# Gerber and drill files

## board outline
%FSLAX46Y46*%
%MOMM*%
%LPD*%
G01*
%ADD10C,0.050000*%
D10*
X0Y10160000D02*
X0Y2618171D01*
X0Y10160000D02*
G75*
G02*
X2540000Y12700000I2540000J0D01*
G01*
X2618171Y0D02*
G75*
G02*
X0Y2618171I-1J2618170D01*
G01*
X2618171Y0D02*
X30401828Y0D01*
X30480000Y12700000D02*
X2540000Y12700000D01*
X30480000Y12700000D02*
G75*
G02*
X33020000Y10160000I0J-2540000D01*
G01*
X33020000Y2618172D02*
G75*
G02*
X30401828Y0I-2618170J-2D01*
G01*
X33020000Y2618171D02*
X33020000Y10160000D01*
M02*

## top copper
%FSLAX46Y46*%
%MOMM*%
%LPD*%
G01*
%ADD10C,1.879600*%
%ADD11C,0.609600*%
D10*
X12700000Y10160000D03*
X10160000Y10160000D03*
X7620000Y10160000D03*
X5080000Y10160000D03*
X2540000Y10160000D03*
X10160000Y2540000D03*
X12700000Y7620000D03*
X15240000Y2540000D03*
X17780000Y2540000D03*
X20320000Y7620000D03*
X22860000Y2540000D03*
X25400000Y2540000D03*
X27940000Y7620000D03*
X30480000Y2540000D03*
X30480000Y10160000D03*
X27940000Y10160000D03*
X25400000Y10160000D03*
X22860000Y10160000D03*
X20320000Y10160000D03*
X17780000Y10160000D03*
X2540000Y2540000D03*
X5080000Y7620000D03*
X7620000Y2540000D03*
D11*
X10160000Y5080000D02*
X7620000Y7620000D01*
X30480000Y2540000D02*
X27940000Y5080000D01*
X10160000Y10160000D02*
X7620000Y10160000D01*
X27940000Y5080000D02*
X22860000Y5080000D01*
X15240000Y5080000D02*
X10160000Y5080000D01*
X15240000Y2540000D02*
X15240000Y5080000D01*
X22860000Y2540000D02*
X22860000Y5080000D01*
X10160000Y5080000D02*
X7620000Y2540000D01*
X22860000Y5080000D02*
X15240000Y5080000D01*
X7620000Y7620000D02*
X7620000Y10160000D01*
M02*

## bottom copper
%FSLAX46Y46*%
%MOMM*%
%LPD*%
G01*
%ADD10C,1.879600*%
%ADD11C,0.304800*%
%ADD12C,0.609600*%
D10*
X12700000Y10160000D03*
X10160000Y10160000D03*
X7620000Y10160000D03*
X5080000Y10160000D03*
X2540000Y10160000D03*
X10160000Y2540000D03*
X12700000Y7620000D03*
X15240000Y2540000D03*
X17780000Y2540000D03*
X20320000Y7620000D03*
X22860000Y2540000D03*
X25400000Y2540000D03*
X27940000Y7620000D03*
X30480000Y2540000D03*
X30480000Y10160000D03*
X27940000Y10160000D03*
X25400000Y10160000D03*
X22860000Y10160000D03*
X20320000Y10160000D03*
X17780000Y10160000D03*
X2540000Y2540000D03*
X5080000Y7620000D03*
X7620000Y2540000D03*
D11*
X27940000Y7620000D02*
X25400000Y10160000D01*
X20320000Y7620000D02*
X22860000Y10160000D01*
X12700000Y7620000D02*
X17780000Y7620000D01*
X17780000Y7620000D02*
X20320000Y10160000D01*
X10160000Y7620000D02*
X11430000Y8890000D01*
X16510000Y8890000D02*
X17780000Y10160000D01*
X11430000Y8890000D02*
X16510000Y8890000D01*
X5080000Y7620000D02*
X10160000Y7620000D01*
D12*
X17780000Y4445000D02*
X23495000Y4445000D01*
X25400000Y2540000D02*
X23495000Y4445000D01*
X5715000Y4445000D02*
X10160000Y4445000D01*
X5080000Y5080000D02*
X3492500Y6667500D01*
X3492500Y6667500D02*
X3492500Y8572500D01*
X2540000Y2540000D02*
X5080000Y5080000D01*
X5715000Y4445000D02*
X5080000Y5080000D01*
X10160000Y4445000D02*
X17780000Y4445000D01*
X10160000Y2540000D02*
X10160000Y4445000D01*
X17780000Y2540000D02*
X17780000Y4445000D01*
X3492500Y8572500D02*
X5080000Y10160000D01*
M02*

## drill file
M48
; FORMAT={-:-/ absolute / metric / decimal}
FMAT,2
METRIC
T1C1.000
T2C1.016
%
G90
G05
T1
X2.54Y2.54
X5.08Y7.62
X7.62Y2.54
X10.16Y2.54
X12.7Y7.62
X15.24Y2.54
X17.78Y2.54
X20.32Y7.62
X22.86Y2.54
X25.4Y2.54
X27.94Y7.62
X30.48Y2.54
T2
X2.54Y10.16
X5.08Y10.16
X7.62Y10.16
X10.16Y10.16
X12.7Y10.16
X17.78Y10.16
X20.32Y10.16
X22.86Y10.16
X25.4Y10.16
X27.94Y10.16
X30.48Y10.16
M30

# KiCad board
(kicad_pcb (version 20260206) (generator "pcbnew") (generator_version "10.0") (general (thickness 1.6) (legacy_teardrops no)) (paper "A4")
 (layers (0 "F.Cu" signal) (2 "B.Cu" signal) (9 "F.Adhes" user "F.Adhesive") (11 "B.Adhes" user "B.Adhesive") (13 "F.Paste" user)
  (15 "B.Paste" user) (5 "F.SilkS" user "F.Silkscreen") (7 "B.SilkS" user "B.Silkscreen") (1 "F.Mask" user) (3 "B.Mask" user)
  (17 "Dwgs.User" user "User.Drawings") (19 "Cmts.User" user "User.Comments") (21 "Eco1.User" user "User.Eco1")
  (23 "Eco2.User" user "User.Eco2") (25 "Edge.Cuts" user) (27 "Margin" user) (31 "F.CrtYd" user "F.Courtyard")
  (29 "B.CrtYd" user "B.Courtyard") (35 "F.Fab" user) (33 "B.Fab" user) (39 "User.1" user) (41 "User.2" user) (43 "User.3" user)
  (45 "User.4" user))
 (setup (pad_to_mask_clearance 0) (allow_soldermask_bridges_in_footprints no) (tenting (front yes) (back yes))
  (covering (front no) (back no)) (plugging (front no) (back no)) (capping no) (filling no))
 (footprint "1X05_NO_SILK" (layer "F.Cu") (at 12.7 -10.16 180)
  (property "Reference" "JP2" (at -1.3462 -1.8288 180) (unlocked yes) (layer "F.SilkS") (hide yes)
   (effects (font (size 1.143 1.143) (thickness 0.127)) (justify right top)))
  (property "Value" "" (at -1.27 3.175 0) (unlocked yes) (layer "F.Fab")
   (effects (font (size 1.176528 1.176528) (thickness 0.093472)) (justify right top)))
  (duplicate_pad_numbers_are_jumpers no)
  (pad "1" thru_hole circle (at 0 0 270) (size 1.8796 1.8796) (drill 1.016) (layers "*.Cu" "*.Mask") (remove_unused_layers no) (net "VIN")
   (solder_mask_margin 0.0762) (thermal_bridge_angle 0))
  (pad "2" thru_hole circle (at 2.54 0 270) (size 1.8796 1.8796) (drill 1.016) (layers "*.Cu" "*.Mask") (remove_unused_layers no)
   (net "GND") (solder_mask_margin 0.0762) (thermal_bridge_angle 0))
  (pad "3" thru_hole circle (at 5.08 0 270) (size 1.8796 1.8796) (drill 1.016) (layers "*.Cu" "*.Mask") (remove_unused_layers no)
   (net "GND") (solder_mask_margin 0.0762) (thermal_bridge_angle 0))
  (pad "4" thru_hole circle (at 7.62 0 270) (size 1.8796 1.8796) (drill 1.016) (layers "*.Cu" "*.Mask") (remove_unused_layers no) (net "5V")
   (solder_mask_margin 0.0762) (thermal_bridge_angle 0))
  (pad "5" thru_hole circle (at 10.16 0 270) (size 1.8796 1.8796) (drill 1.016) (layers "*.Cu" "*.Mask") (remove_unused_layers no)
   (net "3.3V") (solder_mask_margin 0.0762) (thermal_bridge_angle 0)))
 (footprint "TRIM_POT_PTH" (layer "F.Cu") (at 12.7 -5.08)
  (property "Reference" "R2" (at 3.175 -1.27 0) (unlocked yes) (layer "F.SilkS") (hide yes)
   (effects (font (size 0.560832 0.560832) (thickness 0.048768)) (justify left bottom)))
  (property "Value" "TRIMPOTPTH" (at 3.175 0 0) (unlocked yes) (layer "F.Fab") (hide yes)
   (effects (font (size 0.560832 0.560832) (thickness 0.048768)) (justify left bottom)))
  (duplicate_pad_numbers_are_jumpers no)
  (pad "1" thru_hole circle (at -2.54 2.54 180) (size 1.8796 1.8796) (drill 1) (layers "*.Cu" "*.Mask") (remove_unused_layers no) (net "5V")
   (solder_mask_margin 0.0762) (thermal_bridge_angle 0))
  (pad "2" thru_hole circle (at 0 -2.54 180) (size 1.8796 1.8796) (drill 1) (layers "*.Cu" "*.Mask") (remove_unused_layers no) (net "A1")
   (solder_mask_margin 0.0762) (thermal_bridge_angle 0))
  (pad "3" thru_hole circle (at 2.54 2.54 180) (size 1.8796 1.8796) (drill 1) (layers "*.Cu" "*.Mask") (remove_unused_layers no) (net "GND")
   (solder_mask_margin 0.0762) (thermal_bridge_angle 0)))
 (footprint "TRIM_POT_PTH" (layer "F.Cu") (at 20.32 -5.08)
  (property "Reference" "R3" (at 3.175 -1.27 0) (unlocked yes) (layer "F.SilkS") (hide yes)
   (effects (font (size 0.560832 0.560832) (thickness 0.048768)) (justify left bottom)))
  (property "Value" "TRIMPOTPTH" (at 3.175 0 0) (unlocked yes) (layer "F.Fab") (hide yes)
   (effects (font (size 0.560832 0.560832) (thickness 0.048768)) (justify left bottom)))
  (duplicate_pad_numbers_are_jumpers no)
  (pad "1" thru_hole circle (at -2.54 2.54 180) (size 1.8796 1.8796) (drill 1) (layers "*.Cu" "*.Mask") (remove_unused_layers no) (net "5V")
   (solder_mask_margin 0.0762) (thermal_bridge_angle 0))
  (pad "2" thru_hole circle (at 0 -2.54 180) (size 1.8796 1.8796) (drill 1) (layers "*.Cu" "*.Mask") (remove_unused_layers no) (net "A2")
   (solder_mask_margin 0.0762) (thermal_bridge_angle 0))
  (pad "3" thru_hole circle (at 2.54 2.54 180) (size 1.8796 1.8796) (drill 1) (layers "*.Cu" "*.Mask") (remove_unused_layers no) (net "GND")
   (solder_mask_margin 0.0762) (thermal_bridge_angle 0)))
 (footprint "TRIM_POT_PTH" (layer "F.Cu") (at 27.94 -5.08)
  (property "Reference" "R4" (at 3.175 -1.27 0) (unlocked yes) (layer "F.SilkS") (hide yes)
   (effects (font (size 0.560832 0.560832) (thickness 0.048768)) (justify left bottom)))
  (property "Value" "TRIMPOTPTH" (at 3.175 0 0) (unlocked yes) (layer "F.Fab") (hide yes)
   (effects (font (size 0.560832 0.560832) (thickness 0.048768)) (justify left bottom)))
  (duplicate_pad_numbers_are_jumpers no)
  (pad "1" thru_hole circle (at -2.54 2.54 180) (size 1.8796 1.8796) (drill 1) (layers "*.Cu" "*.Mask") (remove_unused_layers no) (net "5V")
   (solder_mask_margin 0.0762) (thermal_bridge_angle 0))
  (pad "2" thru_hole circle (at 0 -2.54 180) (size 1.8796 1.8796) (drill 1) (layers "*.Cu" "*.Mask") (remove_unused_layers no) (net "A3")
   (solder_mask_margin 0.0762) (thermal_bridge_angle 0))
  (pad "3" thru_hole circle (at 2.54 2.54 180) (size 1.8796 1.8796) (drill 1) (layers "*.Cu" "*.Mask") (remove_unused_layers no) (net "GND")
   (solder_mask_margin 0.0762) (thermal_bridge_angle 0)))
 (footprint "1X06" (layer "F.Cu") (at 30.48 -10.16 180)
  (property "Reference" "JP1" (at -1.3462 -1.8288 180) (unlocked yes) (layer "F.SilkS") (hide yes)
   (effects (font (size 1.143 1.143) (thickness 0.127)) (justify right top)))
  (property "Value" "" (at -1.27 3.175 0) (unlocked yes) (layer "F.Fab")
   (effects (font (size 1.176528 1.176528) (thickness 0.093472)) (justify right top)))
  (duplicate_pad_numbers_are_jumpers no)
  (pad "1" thru_hole circle (at 0 0 270) (size 1.8796 1.8796) (drill 1.016) (layers "*.Cu" "*.Mask") (remove_unused_layers no) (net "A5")
   (solder_mask_margin 0.0762) (thermal_bridge_angle 0))
  (pad "2" thru_hole circle (at 2.54 0 270) (size 1.8796 1.8796) (drill 1.016) (layers "*.Cu" "*.Mask") (remove_unused_layers no) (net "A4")
   (solder_mask_margin 0.0762) (thermal_bridge_angle 0))
  (pad "3" thru_hole circle (at 5.08 0 270) (size 1.8796 1.8796) (drill 1.016) (layers "*.Cu" "*.Mask") (remove_unused_layers no) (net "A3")
   (solder_mask_margin 0.0762) (thermal_bridge_angle 0))
  (pad "4" thru_hole circle (at 7.62 0 270) (size 1.8796 1.8796) (drill 1.016) (layers "*.Cu" "*.Mask") (remove_unused_layers no) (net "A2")
   (solder_mask_margin 0.0762) (thermal_bridge_angle 0))
  (pad "5" thru_hole circle (at 10.16 0 270) (size 1.8796 1.8796) (drill 1.016) (layers "*.Cu" "*.Mask") (remove_unused_layers no)
   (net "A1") (solder_mask_margin 0.0762) (thermal_bridge_angle 0))
  (pad "6" thru_hole circle (at 12.7 0 270) (size 1.8796 1.8796) (drill 1.016) (layers "*.Cu" "*.Mask") (remove_unused_layers no) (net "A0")
   (solder_mask_margin 0.0762) (thermal_bridge_angle 0)))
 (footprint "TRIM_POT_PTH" (layer "F.Cu") (at 5.08 -5.08)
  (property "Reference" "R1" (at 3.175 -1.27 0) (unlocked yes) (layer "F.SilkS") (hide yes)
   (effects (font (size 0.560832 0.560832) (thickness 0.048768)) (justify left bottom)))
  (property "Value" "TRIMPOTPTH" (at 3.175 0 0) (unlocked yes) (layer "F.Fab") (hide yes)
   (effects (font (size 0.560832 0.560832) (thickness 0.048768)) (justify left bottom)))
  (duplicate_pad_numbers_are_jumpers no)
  (pad "1" thru_hole circle (at -2.54 2.54 180) (size 1.8796 1.8796) (drill 1) (layers "*.Cu" "*.Mask") (remove_unused_layers no) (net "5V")
   (solder_mask_margin 0.0762) (thermal_bridge_angle 0))
  (pad "2" thru_hole circle (at 0 -2.54 180) (size 1.8796 1.8796) (drill 1) (layers "*.Cu" "*.Mask") (remove_unused_layers no) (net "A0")
   (solder_mask_margin 0.0762) (thermal_bridge_angle 0))
  (pad "3" thru_hole circle (at 2.54 2.54 180) (size 1.8796 1.8796) (drill 1) (layers "*.Cu" "*.Mask") (remove_unused_layers no) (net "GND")
   (solder_mask_margin 0.0762) (thermal_bridge_angle 0)))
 (gr_line (start 0 -10.16) (end 0 -2.618171) (stroke (width 0.05) (type solid)) (layer "Edge.Cuts"))
 (gr_arc (start 0 -10.16) (mid 0.743949 -11.956051) (end 2.54 -12.7) (stroke (width 0.05) (type solid)) (layer "Edge.Cuts"))
 (gr_arc (start 2.618171 0) (mid 0.766845 -0.766845) (end 0 -2.618171) (stroke (width 0.05) (type solid)) (layer "Edge.Cuts"))
 (gr_line (start 2.618171 0) (end 30.401828 0) (stroke (width 0.05) (type solid)) (layer "Edge.Cuts"))
 (gr_line (start 30.48 -12.7) (end 2.54 -12.7) (stroke (width 0.05) (type solid)) (layer "Edge.Cuts"))
 (gr_arc (start 30.48 -12.7) (mid 32.276051 -11.956051) (end 33.02 -10.16) (stroke (width 0.05) (type solid)) (layer "Edge.Cuts"))
 (gr_arc (start 33.02 -2.618172) (mid 32.253155 -0.766845) (end 30.401828 0) (stroke (width 0.05) (type solid)) (layer "Edge.Cuts"))
 (gr_line (start 33.02 -2.618171) (end 33.02 -10.16) (stroke (width 0.05) (type solid)) (layer "Edge.Cuts"))
 (segment (start 27.94 -7.62) (end 25.4 -10.16) (width 0.3048) (layer "B.Cu") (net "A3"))
 (segment (start 20.32 -7.62) (end 22.86 -10.16) (width 0.3048) (layer "B.Cu") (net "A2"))
 (segment (start 12.7 -7.62) (end 17.78 -7.62) (width 0.3048) (layer "B.Cu") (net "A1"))
 (segment (start 17.78 -7.62) (end 20.32 -10.16) (width 0.3048) (layer "B.Cu") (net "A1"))
 (segment (start 10.16 -7.62) (end 11.43 -8.89) (width 0.3048) (layer "B.Cu") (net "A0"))
 (segment (start 16.51 -8.89) (end 17.78 -10.16) (width 0.3048) (layer "B.Cu") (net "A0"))
 (segment (start 11.43 -8.89) (end 16.51 -8.89) (width 0.3048) (layer "B.Cu") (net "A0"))
 (segment (start 5.08 -7.62) (end 10.16 -7.62) (width 0.3048) (layer "B.Cu") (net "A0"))
 (segment (start 17.78 -4.445) (end 23.495 -4.445) (width 0.6096) (layer "B.Cu") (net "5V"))
 (segment (start 25.4 -2.54) (end 23.495 -4.445) (width 0.6096) (layer "B.Cu") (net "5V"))
 (segment (start 5.715 -4.445) (end 10.16 -4.445) (width 0.6096) (layer "B.Cu") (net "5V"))
 (segment (start 5.08 -5.08) (end 3.4925 -6.6675) (width 0.6096) (layer "B.Cu") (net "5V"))
 (segment (start 3.4925 -6.6675) (end 3.4925 -8.5725) (width 0.6096) (layer "B.Cu") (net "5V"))
 (segment (start 2.54 -2.54) (end 5.08 -5.08) (width 0.6096) (layer "B.Cu") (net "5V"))
 (segment (start 5.715 -4.445) (end 5.08 -5.08) (width 0.6096) (layer "B.Cu") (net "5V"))
 (segment (start 10.16 -4.445) (end 17.78 -4.445) (width 0.6096) (layer "B.Cu") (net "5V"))
 (segment (start 10.16 -2.54) (end 10.16 -4.445) (width 0.6096) (layer "B.Cu") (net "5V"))
 (segment (start 17.78 -2.54) (end 17.78 -4.445) (width 0.6096) (layer "B.Cu") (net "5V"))
 (segment (start 3.4925 -8.5725) (end 5.08 -10.16) (width 0.6096) (layer "B.Cu") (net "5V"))
 (segment (start 10.16 -5.08) (end 7.62 -7.62) (width 0.6096) (layer "F.Cu") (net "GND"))
 (segment (start 30.48 -2.54) (end 27.94 -5.08) (width 0.6096) (layer "F.Cu") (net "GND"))
 (segment (start 10.16 -10.16) (end 7.62 -10.16) (width 0.6096) (layer "F.Cu") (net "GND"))
 (segment (start 27.94 -5.08) (end 22.86 -5.08) (width 0.6096) (layer "F.Cu") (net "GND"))
 (segment (start 15.24 -5.08) (end 10.16 -5.08) (width 0.6096) (layer "F.Cu") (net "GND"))
 (segment (start 15.24 -2.54) (end 15.24 -5.08) (width 0.6096) (layer "F.Cu") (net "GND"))
 (segment (start 22.86 -2.54) (end 22.86 -5.08) (width 0.6096) (layer "F.Cu") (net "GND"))
 (segment (start 10.16 -5.08) (end 7.62 -2.54) (width 0.6096) (layer "F.Cu") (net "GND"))
 (segment (start 22.86 -5.08) (end 15.24 -5.08) (width 0.6096) (layer "F.Cu") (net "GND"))
 (segment (start 7.62 -7.62) (end 7.62 -10.16) (width 0.6096) (layer "F.Cu") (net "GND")))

